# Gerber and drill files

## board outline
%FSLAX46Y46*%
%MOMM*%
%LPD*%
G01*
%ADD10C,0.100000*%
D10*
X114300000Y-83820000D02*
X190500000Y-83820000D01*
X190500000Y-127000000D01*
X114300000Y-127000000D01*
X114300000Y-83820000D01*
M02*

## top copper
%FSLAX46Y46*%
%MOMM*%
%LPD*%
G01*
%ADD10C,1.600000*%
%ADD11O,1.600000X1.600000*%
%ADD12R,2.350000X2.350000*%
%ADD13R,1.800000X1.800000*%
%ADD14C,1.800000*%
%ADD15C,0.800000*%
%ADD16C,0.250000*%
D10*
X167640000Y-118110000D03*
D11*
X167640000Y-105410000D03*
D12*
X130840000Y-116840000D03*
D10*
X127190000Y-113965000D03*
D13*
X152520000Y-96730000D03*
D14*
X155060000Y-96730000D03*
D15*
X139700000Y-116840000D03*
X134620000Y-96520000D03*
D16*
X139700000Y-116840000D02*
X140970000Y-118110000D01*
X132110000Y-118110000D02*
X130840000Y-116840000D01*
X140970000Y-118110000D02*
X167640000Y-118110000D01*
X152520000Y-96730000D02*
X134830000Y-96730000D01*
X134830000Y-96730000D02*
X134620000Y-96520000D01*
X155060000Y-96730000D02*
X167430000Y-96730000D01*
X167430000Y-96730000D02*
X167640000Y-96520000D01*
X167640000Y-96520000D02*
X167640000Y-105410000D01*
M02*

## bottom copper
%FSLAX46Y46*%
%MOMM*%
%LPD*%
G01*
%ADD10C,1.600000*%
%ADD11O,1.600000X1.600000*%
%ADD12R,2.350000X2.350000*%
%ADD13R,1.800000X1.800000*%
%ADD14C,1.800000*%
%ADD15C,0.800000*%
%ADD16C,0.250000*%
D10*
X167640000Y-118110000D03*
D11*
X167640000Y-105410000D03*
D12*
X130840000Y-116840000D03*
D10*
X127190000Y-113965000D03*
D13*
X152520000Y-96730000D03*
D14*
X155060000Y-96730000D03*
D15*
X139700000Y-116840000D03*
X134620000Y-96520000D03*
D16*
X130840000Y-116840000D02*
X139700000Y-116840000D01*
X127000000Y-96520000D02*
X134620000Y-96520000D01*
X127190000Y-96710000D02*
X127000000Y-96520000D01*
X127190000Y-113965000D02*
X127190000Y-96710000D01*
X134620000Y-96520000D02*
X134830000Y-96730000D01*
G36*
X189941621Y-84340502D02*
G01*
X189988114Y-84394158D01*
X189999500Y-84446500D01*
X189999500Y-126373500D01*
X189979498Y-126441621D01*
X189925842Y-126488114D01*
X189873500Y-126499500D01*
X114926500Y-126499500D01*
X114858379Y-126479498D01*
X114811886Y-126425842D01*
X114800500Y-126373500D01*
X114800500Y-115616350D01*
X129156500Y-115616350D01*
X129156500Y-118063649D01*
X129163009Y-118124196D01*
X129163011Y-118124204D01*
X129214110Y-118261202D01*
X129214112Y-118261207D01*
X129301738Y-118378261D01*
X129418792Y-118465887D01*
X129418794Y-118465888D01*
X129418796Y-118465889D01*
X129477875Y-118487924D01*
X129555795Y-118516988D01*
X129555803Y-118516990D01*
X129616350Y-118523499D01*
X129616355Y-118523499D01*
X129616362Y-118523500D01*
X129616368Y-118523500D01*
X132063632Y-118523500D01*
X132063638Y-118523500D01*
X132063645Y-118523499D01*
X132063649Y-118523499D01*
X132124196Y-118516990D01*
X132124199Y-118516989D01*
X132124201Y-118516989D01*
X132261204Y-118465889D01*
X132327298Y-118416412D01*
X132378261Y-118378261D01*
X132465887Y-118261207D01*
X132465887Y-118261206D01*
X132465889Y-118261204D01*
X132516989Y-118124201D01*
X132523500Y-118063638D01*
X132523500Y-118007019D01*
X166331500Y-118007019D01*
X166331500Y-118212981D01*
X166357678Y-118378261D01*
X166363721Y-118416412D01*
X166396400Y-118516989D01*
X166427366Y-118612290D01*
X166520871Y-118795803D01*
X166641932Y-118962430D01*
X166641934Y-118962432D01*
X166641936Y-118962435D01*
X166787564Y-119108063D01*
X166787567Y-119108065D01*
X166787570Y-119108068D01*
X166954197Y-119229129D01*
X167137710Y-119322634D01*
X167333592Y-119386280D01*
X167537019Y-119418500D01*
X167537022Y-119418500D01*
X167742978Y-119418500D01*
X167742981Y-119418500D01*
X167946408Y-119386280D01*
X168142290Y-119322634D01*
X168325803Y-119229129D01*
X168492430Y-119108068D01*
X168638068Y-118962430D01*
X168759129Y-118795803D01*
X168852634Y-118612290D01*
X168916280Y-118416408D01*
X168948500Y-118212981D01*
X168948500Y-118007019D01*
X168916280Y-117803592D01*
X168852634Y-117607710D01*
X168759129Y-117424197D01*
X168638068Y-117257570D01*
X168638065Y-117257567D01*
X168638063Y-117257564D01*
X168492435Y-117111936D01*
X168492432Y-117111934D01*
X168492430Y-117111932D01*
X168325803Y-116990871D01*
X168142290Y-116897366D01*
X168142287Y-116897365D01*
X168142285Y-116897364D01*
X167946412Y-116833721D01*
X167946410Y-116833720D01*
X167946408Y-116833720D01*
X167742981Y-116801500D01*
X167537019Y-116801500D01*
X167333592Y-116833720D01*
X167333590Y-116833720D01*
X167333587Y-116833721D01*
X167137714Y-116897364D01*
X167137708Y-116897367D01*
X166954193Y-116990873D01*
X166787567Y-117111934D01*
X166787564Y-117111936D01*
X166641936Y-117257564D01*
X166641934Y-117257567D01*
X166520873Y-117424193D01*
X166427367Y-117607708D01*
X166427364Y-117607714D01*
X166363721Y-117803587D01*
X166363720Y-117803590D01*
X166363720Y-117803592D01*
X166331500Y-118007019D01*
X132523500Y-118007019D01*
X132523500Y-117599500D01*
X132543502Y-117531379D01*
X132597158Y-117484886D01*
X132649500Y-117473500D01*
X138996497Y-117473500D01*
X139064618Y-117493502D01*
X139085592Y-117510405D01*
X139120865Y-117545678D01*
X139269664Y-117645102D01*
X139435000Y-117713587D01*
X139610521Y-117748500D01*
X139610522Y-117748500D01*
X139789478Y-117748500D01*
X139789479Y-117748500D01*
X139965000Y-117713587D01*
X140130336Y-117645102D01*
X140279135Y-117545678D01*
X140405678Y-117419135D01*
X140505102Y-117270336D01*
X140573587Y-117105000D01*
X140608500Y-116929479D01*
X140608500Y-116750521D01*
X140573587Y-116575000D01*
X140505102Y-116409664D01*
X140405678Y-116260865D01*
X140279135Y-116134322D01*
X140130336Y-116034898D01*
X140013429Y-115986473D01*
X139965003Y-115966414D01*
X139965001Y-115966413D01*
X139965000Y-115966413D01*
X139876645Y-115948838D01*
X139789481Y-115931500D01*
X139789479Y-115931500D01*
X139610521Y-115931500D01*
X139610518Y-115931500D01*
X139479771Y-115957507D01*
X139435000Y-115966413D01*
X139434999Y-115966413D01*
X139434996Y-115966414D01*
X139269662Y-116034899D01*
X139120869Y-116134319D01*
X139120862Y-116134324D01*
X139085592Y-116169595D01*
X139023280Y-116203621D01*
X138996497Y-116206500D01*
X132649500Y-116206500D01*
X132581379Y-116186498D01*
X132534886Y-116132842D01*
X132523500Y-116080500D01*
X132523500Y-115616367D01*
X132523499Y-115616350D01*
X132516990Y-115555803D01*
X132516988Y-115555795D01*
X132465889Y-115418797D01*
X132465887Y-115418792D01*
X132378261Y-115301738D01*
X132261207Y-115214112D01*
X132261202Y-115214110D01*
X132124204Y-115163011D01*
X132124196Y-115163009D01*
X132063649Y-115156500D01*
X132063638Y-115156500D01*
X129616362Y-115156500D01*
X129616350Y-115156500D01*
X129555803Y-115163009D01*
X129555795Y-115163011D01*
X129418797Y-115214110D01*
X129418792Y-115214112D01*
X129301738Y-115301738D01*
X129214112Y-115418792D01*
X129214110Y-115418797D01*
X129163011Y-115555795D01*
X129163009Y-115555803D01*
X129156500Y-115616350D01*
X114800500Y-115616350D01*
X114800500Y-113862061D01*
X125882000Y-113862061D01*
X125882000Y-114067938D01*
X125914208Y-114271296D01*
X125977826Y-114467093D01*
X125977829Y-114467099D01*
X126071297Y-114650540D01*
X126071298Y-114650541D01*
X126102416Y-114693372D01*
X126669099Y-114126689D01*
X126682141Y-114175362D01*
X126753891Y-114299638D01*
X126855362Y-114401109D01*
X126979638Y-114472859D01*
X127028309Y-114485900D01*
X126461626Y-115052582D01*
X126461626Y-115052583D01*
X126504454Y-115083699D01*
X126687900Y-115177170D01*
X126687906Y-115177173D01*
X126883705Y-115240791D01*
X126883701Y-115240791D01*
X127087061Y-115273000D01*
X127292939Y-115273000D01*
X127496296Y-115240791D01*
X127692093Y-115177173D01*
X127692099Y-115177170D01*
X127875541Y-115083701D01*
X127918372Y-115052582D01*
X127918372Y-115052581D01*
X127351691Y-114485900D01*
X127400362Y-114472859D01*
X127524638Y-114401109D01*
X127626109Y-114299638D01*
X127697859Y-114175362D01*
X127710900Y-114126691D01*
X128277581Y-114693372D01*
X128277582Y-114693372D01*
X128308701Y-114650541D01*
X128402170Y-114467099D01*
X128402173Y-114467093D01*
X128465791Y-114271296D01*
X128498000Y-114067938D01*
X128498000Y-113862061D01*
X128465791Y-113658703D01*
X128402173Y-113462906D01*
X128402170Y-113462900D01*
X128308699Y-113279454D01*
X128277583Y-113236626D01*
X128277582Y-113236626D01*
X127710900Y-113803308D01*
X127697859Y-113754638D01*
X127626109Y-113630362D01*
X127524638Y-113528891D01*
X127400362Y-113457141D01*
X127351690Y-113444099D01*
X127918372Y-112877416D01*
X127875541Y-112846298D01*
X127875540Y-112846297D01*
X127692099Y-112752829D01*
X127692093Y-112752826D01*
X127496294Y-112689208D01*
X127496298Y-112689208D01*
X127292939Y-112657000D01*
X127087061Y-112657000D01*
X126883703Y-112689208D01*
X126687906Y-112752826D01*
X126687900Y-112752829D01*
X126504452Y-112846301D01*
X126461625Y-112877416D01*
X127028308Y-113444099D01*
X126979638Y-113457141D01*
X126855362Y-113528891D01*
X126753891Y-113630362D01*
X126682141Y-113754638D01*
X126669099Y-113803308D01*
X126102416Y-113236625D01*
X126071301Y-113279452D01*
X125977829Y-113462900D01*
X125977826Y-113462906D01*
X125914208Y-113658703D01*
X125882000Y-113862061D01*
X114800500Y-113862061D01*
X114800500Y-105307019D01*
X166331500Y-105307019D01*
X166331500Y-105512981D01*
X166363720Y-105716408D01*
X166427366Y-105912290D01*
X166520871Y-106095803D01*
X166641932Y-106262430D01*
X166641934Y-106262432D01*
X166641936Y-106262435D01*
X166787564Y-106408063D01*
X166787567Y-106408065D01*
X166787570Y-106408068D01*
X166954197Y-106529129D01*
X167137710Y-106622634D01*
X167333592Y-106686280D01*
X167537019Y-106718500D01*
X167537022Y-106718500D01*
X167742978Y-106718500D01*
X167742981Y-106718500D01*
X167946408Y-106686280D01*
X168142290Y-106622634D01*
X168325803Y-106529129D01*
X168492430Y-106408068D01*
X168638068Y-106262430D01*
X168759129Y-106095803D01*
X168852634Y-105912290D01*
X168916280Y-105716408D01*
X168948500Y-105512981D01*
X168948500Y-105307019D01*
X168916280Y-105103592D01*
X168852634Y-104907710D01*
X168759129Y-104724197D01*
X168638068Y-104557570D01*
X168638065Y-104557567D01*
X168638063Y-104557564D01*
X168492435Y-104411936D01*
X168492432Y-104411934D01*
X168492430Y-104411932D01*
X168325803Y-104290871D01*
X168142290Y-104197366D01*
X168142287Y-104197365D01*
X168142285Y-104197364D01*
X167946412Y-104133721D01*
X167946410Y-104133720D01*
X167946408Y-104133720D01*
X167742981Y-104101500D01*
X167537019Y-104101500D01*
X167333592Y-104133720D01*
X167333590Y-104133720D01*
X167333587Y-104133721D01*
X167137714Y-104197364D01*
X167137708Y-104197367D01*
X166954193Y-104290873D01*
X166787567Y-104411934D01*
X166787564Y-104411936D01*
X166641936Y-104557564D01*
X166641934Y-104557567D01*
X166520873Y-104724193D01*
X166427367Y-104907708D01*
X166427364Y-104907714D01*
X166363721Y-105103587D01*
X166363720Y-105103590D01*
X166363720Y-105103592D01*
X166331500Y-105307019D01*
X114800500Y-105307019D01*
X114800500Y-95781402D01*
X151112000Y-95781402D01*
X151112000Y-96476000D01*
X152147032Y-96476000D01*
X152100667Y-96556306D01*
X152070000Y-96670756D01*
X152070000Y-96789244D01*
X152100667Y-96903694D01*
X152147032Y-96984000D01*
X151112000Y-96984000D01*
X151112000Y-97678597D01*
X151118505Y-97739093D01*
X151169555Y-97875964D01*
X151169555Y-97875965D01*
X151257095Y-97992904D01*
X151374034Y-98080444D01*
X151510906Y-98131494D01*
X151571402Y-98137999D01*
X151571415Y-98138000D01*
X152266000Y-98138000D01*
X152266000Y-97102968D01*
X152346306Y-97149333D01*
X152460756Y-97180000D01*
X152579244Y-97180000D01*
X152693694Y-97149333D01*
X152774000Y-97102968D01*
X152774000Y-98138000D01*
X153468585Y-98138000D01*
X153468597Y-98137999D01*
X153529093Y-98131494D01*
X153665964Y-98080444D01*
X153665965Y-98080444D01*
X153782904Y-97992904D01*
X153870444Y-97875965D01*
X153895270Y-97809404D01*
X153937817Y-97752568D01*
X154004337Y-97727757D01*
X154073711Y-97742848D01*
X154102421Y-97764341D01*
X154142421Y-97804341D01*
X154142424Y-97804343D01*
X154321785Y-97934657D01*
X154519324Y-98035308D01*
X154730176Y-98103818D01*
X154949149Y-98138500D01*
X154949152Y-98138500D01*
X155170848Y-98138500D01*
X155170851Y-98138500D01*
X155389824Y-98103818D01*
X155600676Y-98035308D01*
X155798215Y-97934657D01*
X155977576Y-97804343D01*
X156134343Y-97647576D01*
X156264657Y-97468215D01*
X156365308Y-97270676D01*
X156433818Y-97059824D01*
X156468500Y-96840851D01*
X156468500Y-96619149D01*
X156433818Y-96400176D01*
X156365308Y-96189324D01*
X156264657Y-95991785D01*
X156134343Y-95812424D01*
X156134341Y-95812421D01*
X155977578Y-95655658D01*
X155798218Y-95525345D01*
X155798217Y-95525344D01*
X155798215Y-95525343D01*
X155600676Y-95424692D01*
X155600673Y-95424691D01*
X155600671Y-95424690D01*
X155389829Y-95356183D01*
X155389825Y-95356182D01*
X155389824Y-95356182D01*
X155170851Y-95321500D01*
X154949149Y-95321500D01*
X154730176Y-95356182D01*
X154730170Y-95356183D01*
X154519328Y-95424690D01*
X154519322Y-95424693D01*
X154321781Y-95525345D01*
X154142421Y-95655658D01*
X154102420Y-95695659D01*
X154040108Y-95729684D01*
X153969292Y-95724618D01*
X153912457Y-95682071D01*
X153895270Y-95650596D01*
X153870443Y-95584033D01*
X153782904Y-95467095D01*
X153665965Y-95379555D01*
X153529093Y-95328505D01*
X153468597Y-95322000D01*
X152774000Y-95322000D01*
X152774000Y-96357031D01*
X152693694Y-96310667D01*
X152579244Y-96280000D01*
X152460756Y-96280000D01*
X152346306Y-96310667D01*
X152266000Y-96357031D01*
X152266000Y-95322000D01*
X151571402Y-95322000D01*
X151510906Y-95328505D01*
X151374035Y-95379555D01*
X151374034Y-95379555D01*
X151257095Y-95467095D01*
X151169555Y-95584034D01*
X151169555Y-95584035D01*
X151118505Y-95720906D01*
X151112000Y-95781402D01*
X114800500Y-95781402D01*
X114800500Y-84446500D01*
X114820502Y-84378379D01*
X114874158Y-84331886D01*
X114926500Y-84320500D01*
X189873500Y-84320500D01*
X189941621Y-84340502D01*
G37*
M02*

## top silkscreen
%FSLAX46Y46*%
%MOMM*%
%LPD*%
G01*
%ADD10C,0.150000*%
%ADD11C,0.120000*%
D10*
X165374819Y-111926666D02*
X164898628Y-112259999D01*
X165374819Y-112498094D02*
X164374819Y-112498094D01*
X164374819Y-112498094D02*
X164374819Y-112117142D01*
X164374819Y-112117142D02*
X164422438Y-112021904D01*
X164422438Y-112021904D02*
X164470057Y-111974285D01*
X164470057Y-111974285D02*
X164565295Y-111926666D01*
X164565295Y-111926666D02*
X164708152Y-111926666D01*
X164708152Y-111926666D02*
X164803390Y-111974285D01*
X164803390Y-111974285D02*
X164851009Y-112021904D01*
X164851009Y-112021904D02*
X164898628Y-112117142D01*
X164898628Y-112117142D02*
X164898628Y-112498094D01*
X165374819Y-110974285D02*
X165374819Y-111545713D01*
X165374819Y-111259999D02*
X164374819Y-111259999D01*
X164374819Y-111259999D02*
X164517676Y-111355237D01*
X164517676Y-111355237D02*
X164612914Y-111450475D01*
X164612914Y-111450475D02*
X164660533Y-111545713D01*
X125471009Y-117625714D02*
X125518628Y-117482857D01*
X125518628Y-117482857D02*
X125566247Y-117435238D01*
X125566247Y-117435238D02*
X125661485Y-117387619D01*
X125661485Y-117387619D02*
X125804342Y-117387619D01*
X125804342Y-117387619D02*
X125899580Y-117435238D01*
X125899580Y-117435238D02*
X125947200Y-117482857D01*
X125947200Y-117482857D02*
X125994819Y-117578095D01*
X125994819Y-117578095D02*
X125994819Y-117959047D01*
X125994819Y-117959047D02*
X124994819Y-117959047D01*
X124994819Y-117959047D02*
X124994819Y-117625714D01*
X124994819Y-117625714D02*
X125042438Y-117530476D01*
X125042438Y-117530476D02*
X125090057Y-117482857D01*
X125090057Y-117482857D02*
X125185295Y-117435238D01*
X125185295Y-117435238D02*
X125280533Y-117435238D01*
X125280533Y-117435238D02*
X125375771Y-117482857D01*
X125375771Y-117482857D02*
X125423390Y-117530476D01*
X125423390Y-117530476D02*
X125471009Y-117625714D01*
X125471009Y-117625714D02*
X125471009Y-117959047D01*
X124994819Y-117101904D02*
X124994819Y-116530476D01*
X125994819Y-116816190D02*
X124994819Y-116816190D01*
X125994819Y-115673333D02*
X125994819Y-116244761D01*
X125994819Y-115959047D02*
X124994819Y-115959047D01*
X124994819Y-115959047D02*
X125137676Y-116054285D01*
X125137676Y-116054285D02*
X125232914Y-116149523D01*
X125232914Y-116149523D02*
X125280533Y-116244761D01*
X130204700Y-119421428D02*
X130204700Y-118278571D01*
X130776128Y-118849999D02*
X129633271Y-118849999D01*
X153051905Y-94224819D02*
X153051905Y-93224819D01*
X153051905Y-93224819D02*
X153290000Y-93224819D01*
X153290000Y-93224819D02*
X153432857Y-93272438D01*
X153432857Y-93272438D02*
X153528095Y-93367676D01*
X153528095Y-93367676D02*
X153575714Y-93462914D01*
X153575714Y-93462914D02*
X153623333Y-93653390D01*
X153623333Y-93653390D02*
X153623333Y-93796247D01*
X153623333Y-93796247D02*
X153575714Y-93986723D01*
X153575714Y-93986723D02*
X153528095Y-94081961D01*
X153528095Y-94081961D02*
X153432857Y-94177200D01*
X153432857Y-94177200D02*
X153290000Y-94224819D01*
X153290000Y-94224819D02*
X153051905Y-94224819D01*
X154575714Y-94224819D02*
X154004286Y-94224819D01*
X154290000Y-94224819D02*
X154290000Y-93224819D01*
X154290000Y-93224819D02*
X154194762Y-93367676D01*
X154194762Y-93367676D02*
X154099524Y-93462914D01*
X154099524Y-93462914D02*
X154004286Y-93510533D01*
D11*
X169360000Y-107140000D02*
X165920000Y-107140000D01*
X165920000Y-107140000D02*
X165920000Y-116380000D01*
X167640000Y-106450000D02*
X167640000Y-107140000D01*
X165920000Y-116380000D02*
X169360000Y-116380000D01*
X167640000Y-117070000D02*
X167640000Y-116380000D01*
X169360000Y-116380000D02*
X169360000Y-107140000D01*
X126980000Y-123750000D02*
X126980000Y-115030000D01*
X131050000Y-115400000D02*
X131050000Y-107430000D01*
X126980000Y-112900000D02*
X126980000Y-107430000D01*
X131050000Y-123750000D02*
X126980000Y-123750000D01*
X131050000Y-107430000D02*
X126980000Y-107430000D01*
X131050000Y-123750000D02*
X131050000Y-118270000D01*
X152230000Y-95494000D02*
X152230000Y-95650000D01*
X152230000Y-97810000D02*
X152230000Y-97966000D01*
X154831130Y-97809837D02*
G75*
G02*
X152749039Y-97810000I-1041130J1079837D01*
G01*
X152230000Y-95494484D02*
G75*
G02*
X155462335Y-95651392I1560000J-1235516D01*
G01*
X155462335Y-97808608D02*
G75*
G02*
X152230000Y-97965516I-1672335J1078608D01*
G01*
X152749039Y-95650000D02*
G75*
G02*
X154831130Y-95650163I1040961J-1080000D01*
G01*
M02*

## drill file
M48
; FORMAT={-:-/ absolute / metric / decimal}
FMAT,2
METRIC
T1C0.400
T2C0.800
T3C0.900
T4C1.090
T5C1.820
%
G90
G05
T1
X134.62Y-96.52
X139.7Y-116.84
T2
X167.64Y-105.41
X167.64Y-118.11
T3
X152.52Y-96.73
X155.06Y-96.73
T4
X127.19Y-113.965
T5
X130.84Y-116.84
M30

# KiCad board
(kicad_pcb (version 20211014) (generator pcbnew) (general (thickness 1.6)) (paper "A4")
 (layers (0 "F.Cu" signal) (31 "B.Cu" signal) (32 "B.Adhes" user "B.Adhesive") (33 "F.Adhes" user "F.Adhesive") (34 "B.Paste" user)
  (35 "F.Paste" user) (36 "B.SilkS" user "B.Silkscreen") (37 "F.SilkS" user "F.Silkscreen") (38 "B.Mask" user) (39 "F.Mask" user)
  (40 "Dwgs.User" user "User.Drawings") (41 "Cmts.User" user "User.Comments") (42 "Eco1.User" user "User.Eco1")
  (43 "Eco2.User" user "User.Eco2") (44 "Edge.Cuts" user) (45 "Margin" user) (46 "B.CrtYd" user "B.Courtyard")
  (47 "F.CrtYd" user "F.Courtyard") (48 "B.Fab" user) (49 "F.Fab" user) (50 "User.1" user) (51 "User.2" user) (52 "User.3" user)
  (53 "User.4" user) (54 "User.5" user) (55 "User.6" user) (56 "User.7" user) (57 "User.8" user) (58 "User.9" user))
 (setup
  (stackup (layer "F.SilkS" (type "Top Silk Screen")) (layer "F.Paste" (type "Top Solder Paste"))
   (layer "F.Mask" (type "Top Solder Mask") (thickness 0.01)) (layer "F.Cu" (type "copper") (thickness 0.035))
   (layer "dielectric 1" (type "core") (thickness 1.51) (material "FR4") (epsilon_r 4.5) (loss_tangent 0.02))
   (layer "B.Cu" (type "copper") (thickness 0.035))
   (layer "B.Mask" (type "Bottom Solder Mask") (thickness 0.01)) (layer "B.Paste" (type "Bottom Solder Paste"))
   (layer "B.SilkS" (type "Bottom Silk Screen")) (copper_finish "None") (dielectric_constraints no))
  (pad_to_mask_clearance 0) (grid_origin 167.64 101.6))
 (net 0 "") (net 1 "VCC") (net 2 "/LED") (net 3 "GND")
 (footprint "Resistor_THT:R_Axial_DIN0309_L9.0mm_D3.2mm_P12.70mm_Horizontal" (layer "F.Cu") (at 167.64 118.11 90)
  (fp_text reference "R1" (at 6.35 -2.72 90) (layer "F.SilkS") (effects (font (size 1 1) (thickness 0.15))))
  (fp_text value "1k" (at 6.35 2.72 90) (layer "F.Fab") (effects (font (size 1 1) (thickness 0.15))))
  (fp_line (start 10.97 1.72) (end 10.97 -1.72) (layer "F.SilkS") (width 0.12))
  (fp_line (start 10.97 -1.72) (end 1.73 -1.72) (layer "F.SilkS") (width 0.12))
  (fp_line (start 11.66 0) (end 10.97 0) (layer "F.SilkS") (width 0.12))
  (fp_line (start 1.73 -1.72) (end 1.73 1.72) (layer "F.SilkS") (width 0.12))
  (fp_line (start 1.04 0) (end 1.73 0) (layer "F.SilkS") (width 0.12))
  (fp_line (start 1.73 1.72) (end 10.97 1.72) (layer "F.SilkS") (width 0.12))
  (pad "1" thru_hole circle (at 0 0 90) (size 1.6 1.6) (drill 0.8) (layers *.Cu *.Mask) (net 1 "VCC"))
  (pad "2" thru_hole oval (at 12.7 0 90) (size 1.6 1.6) (drill 0.8) (layers *.Cu *.Mask) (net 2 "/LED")))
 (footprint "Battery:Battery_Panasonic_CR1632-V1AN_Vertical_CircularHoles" (layer "F.Cu") (at 130.84 116.84 90)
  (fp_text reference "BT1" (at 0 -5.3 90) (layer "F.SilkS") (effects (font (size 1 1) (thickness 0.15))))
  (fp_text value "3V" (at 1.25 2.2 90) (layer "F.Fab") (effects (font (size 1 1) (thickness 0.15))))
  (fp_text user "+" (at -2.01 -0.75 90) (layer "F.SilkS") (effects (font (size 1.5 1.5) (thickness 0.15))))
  (fp_line (start -6.91 -3.86) (end 1.81 -3.86) (layer "F.SilkS") (width 0.12))
  (fp_line (start 1.44 0.21) (end 9.41 0.21) (layer "F.SilkS") (width 0.12))
  (fp_line (start 3.94 -3.86) (end 9.41 -3.86) (layer "F.SilkS") (width 0.12))
  (fp_line (start -6.91 0.21) (end -6.91 -3.86) (layer "F.SilkS") (width 0.12))
  (fp_line (start 9.41 0.21) (end 9.41 -3.86) (layer "F.SilkS") (width 0.12))
  (fp_line (start -6.91 0.21) (end -1.43 0.21) (layer "F.SilkS") (width 0.12))
  (pad "1" thru_hole rect (at 0 0 180) (size 2.35 2.35) (drill 1.82) (layers *.Cu *.Mask) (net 1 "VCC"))
  (pad "2" thru_hole circle (at 2.875 -3.65 90) (size 1.6 1.6) (drill 1.09) (layers *.Cu *.Mask) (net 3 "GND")))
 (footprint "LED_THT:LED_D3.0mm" (layer "F.Cu") (at 152.52 96.73)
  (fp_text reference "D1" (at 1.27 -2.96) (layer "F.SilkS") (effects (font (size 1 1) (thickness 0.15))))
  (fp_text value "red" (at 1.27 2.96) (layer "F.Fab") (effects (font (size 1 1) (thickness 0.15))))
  (fp_line (start -0.29 -1.236) (end -0.29 -1.08) (layer "F.SilkS") (width 0.12))
  (fp_line (start -0.29 1.08) (end -0.29 1.236) (layer "F.SilkS") (width 0.12))
  (fp_arc (start 2.31113 1.079837) (mid 1.270117 1.5) (end 0.229039 1.08) (layer "F.SilkS") (width 0.12))
  (fp_arc (start -0.29 -1.235516) (mid 1.366487 -1.987659) (end 2.942335 -1.078608) (layer "F.SilkS") (width 0.12))
  (fp_arc (start 2.942335 1.078608) (mid 1.366487 1.987659) (end -0.29 1.235516) (layer "F.SilkS") (width 0.12))
  (fp_arc (start 0.229039 -1.08) (mid 1.270117 -1.5) (end 2.31113 -1.079837) (layer "F.SilkS") (width 0.12))
  (pad "1" thru_hole rect (at 0 0) (size 1.8 1.8) (drill 0.9) (layers *.Cu *.Mask) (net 3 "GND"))
  (pad "2" thru_hole circle (at 2.54 0) (size 1.8 1.8) (drill 0.9) (layers *.Cu *.Mask) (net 2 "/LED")))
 (gr_rect (start 114.3 127) (end 190.5 83.82) (layer "Edge.Cuts") (width 0.1) (fill none))
 (segment (start 139.7 116.84) (end 140.97 118.11) (width 0.25) (layer "F.Cu") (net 1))
 (segment (start 132.11 118.11) (end 130.84 116.84) (width 0.25) (layer "F.Cu") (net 1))
 (segment (start 140.97 118.11) (end 167.64 118.11) (width 0.25) (layer "F.Cu") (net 1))
 (via (at 139.7 116.84) (size 0.8) (drill 0.4) (layers "F.Cu" "B.Cu") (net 1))
 (segment (start 130.84 116.84) (end 139.7 116.84) (width 0.25) (layer "B.Cu") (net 1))
 (segment (start 152.52 96.73) (end 134.83 96.73) (width 0.25) (layer "F.Cu") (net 3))
 (segment (start 134.83 96.73) (end 134.62 96.52) (width 0.25) (layer "F.Cu") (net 3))
 (via (at 134.62 96.52) (size 0.8) (drill 0.4) (layers "F.Cu" "B.Cu") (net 3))
 (segment (start 127 96.52) (end 134.62 96.52) (width 0.25) (layer "B.Cu") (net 3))
 (segment (start 127.19 96.71) (end 127 96.52) (width 0.25) (layer "B.Cu") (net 3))
 (segment (start 127.19 113.965) (end 127.19 96.71) (width 0.25) (layer "B.Cu") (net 3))
 (segment (start 134.62 96.52) (end 134.83 96.73) (width 0.25) (layer "B.Cu") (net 3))
 (segment (start 155.06 96.73) (end 167.43 96.73) (width 0.25) (layer "F.Cu") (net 2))
 (segment (start 167.43 96.73) (end 167.64 96.52) (width 0.25) (layer "F.Cu") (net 2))
 (segment (start 167.64 96.52) (end 167.64 105.41) (width 0.25) (layer "F.Cu") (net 2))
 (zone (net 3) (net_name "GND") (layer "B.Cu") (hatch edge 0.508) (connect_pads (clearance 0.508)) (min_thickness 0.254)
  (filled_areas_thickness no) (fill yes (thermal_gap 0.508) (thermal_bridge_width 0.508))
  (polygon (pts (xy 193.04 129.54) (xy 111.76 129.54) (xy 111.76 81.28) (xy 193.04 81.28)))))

